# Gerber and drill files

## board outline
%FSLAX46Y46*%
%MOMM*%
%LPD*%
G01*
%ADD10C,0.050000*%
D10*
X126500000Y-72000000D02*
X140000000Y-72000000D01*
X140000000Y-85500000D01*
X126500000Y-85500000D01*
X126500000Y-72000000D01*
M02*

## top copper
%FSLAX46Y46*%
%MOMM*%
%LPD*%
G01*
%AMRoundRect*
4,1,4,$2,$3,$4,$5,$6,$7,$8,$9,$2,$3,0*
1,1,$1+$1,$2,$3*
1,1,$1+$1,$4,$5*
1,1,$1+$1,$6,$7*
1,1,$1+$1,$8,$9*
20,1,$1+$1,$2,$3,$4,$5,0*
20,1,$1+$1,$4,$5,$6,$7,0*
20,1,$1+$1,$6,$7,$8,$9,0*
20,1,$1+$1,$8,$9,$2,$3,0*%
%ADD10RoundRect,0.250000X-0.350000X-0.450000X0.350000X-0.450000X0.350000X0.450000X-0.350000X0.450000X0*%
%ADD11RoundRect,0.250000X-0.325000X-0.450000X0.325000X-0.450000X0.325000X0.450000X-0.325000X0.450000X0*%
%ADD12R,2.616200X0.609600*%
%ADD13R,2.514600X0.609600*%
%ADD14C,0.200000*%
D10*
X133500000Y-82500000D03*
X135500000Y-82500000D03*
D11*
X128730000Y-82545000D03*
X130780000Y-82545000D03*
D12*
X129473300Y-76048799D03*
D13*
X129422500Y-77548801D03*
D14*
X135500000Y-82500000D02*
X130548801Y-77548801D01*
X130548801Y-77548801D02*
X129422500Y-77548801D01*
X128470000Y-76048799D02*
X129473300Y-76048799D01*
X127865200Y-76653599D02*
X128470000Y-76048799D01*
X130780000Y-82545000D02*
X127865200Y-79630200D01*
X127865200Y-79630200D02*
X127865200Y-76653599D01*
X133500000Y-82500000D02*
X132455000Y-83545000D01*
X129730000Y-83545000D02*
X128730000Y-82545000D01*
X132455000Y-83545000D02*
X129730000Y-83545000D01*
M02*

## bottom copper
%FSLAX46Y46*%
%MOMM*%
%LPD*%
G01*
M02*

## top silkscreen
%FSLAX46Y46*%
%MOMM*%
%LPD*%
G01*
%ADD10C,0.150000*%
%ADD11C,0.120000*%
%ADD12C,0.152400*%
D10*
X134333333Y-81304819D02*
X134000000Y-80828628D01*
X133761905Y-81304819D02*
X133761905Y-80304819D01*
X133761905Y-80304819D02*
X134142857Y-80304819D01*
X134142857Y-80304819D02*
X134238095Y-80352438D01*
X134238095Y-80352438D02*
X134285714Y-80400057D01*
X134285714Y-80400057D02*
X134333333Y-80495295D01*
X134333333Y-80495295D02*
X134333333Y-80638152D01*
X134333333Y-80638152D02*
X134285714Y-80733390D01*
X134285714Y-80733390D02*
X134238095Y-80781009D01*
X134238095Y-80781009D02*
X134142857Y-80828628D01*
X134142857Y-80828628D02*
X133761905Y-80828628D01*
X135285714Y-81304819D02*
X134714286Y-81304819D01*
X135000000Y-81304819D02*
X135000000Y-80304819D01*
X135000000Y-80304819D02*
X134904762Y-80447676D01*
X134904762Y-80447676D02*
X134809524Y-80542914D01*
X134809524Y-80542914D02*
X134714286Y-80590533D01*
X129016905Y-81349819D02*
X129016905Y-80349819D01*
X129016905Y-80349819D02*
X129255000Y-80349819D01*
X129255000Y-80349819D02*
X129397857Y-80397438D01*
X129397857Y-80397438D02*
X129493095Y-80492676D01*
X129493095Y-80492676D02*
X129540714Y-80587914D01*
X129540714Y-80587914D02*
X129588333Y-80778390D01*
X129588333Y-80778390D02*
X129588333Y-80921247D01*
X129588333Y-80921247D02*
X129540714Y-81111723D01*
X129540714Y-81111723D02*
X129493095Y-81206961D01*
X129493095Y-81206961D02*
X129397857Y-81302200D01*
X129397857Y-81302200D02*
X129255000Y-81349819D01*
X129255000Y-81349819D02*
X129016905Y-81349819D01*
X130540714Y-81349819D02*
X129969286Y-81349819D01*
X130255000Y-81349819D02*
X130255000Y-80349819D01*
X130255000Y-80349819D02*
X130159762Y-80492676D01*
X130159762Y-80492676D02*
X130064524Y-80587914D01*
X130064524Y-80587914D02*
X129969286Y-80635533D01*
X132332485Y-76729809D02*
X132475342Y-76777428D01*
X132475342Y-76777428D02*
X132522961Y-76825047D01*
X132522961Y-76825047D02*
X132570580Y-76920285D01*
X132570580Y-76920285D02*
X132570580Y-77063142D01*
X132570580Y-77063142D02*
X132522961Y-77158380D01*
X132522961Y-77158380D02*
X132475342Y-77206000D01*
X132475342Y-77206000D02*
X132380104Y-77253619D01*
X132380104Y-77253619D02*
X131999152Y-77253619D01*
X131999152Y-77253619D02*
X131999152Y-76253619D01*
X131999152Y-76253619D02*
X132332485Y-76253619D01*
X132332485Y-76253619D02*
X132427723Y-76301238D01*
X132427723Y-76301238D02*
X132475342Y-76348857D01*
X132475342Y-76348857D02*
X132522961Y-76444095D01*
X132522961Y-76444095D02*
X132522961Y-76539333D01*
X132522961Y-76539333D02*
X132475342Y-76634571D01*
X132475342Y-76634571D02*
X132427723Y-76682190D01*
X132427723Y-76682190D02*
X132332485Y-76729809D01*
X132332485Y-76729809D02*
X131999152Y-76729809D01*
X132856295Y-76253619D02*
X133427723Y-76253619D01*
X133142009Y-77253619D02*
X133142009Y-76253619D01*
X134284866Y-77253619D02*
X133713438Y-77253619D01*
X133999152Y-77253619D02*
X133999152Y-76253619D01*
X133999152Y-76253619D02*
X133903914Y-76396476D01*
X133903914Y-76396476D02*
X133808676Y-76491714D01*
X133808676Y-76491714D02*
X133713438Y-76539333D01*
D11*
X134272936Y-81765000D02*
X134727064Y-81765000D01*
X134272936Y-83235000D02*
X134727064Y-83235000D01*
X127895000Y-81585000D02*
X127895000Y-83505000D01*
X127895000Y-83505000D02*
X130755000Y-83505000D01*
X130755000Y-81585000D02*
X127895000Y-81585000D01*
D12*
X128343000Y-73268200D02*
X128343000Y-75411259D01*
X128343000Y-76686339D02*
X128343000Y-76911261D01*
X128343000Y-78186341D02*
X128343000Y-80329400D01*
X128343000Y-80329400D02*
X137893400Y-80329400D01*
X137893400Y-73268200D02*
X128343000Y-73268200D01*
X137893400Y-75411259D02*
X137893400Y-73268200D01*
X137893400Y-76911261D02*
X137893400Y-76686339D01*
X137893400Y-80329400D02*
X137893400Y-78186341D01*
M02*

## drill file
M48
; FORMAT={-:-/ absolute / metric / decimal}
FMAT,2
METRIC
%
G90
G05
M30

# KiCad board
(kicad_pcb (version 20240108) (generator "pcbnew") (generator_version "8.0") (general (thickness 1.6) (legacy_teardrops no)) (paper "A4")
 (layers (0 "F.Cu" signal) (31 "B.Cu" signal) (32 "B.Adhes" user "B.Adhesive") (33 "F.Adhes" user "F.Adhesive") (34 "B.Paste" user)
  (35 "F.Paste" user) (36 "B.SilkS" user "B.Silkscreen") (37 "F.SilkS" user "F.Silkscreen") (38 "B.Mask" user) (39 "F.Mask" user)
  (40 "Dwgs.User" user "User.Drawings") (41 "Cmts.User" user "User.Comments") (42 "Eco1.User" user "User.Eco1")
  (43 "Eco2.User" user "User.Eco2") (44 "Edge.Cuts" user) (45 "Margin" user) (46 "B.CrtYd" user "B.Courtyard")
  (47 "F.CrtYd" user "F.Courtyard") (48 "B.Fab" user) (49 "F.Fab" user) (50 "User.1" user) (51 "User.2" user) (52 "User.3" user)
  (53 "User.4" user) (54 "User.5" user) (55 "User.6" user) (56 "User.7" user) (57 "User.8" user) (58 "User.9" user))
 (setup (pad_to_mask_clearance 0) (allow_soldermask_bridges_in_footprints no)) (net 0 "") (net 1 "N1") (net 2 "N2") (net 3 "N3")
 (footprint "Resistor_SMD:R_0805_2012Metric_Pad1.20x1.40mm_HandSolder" (layer "F.Cu") (at 134.5 82.5)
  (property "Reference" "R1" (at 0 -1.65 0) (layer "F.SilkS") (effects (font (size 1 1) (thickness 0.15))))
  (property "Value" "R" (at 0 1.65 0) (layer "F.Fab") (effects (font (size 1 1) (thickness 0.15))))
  (fp_line (start -0.227064 -0.735) (end 0.227064 -0.735) (stroke (width 0.12) (type solid)) (layer "F.SilkS"))
  (fp_line (start -0.227064 0.735) (end 0.227064 0.735) (stroke (width 0.12) (type solid)) (layer "F.SilkS"))
  (pad "1" smd roundrect (at -1 0) (size 1.2 1.4) (layers "F.Cu" "F.Paste" "F.Mask") (roundrect_rratio 0.208333) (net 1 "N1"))
  (pad "2" smd roundrect (at 1 0) (size 1.2 1.4) (layers "F.Cu" "F.Paste" "F.Mask") (roundrect_rratio 0.208333) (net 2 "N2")))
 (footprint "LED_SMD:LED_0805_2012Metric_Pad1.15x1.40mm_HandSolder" (layer "F.Cu") (at 129.755 82.545)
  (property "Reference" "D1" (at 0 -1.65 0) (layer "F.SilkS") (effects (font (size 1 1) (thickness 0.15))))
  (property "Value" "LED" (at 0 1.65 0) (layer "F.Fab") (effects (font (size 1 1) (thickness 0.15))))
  (fp_line (start -1.86 -0.96) (end -1.86 0.96) (stroke (width 0.12) (type solid)) (layer "F.SilkS"))
  (fp_line (start -1.86 0.96) (end 1 0.96) (stroke (width 0.12) (type solid)) (layer "F.SilkS"))
  (fp_line (start 1 -0.96) (end -1.86 -0.96) (stroke (width 0.12) (type solid)) (layer "F.SilkS"))
  (pad "1" smd roundrect (at -1.025 0) (size 1.15 1.4) (layers "F.Cu" "F.Paste" "F.Mask") (roundrect_rratio 0.217391) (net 1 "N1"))
  (pad "2" smd roundrect (at 1.025 0) (size 1.15 1.4) (layers "F.Cu" "F.Paste" "F.Mask") (roundrect_rratio 0.217391) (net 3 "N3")))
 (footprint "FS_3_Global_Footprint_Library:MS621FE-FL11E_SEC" (layer "F.Cu") (at 133.1182 76.7988)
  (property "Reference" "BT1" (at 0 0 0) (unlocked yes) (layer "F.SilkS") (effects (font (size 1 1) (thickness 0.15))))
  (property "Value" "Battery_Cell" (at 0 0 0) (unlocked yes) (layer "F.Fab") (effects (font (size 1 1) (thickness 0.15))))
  (fp_line (start -4.7752 -3.5306) (end -4.7752 -1.387541) (stroke (width 0.1524) (type solid)) (layer "F.SilkS"))
  (fp_line (start -4.7752 -0.112461) (end -4.7752 0.112461) (stroke (width 0.1524) (type solid)) (layer "F.SilkS"))
  (fp_line (start -4.7752 1.387541) (end -4.7752 3.5306) (stroke (width 0.1524) (type solid)) (layer "F.SilkS"))
  (fp_line (start -4.7752 3.5306) (end 4.7752 3.5306) (stroke (width 0.1524) (type solid)) (layer "F.SilkS"))
  (fp_line (start 4.7752 -3.5306) (end -4.7752 -3.5306) (stroke (width 0.1524) (type solid)) (layer "F.SilkS"))
  (fp_line (start 4.7752 -1.387541) (end 4.7752 -3.5306) (stroke (width 0.1524) (type solid)) (layer "F.SilkS"))
  (fp_line (start 4.7752 0.112461) (end 4.7752 -0.112461) (stroke (width 0.1524) (type solid)) (layer "F.SilkS"))
  (fp_line (start 4.7752 3.5306) (end 4.7752 1.387541) (stroke (width 0.1524) (type solid)) (layer "F.SilkS"))
  (pad "1" smd rect (at -3.6449 -0.750001) (size 2.6162 0.6096) (layers "F.Cu" "F.Paste" "F.Mask") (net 3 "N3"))
  (pad "2" smd rect (at -3.6957 0.750001) (size 2.5146 0.6096) (layers "F.Cu" "F.Paste" "F.Mask") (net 2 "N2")))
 (gr_rect (start 126.5 72) (end 140 85.5) (stroke (width 0.05) (type default)) (fill none) (layer "Edge.Cuts"))
 (segment (start 135.5 82.5) (end 130.548801 77.548801) (width 0.2) (layer "F.Cu") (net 2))
 (segment (start 130.548801 77.548801) (end 129.4225 77.548801) (width 0.2) (layer "F.Cu") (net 2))
 (segment (start 128.47 76.048799) (end 129.4733 76.048799) (width 0.2) (layer "F.Cu") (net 3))
 (segment (start 127.8652 76.653599) (end 128.47 76.048799) (width 0.2) (layer "F.Cu") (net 3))
 (segment (start 130.78 82.545) (end 127.8652 79.6302) (width 0.2) (layer "F.Cu") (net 3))
 (segment (start 127.8652 79.6302) (end 127.8652 76.653599) (width 0.2) (layer "F.Cu") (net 3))
 (segment (start 133.5 82.5) (end 132.455 83.545) (width 0.2) (layer "F.Cu") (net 1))
 (segment (start 129.73 83.545) (end 128.73 82.545) (width 0.2) (layer "F.Cu") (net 1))
 (segment (start 132.455 83.545) (end 129.73 83.545) (width 0.2) (layer "F.Cu") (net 1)))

